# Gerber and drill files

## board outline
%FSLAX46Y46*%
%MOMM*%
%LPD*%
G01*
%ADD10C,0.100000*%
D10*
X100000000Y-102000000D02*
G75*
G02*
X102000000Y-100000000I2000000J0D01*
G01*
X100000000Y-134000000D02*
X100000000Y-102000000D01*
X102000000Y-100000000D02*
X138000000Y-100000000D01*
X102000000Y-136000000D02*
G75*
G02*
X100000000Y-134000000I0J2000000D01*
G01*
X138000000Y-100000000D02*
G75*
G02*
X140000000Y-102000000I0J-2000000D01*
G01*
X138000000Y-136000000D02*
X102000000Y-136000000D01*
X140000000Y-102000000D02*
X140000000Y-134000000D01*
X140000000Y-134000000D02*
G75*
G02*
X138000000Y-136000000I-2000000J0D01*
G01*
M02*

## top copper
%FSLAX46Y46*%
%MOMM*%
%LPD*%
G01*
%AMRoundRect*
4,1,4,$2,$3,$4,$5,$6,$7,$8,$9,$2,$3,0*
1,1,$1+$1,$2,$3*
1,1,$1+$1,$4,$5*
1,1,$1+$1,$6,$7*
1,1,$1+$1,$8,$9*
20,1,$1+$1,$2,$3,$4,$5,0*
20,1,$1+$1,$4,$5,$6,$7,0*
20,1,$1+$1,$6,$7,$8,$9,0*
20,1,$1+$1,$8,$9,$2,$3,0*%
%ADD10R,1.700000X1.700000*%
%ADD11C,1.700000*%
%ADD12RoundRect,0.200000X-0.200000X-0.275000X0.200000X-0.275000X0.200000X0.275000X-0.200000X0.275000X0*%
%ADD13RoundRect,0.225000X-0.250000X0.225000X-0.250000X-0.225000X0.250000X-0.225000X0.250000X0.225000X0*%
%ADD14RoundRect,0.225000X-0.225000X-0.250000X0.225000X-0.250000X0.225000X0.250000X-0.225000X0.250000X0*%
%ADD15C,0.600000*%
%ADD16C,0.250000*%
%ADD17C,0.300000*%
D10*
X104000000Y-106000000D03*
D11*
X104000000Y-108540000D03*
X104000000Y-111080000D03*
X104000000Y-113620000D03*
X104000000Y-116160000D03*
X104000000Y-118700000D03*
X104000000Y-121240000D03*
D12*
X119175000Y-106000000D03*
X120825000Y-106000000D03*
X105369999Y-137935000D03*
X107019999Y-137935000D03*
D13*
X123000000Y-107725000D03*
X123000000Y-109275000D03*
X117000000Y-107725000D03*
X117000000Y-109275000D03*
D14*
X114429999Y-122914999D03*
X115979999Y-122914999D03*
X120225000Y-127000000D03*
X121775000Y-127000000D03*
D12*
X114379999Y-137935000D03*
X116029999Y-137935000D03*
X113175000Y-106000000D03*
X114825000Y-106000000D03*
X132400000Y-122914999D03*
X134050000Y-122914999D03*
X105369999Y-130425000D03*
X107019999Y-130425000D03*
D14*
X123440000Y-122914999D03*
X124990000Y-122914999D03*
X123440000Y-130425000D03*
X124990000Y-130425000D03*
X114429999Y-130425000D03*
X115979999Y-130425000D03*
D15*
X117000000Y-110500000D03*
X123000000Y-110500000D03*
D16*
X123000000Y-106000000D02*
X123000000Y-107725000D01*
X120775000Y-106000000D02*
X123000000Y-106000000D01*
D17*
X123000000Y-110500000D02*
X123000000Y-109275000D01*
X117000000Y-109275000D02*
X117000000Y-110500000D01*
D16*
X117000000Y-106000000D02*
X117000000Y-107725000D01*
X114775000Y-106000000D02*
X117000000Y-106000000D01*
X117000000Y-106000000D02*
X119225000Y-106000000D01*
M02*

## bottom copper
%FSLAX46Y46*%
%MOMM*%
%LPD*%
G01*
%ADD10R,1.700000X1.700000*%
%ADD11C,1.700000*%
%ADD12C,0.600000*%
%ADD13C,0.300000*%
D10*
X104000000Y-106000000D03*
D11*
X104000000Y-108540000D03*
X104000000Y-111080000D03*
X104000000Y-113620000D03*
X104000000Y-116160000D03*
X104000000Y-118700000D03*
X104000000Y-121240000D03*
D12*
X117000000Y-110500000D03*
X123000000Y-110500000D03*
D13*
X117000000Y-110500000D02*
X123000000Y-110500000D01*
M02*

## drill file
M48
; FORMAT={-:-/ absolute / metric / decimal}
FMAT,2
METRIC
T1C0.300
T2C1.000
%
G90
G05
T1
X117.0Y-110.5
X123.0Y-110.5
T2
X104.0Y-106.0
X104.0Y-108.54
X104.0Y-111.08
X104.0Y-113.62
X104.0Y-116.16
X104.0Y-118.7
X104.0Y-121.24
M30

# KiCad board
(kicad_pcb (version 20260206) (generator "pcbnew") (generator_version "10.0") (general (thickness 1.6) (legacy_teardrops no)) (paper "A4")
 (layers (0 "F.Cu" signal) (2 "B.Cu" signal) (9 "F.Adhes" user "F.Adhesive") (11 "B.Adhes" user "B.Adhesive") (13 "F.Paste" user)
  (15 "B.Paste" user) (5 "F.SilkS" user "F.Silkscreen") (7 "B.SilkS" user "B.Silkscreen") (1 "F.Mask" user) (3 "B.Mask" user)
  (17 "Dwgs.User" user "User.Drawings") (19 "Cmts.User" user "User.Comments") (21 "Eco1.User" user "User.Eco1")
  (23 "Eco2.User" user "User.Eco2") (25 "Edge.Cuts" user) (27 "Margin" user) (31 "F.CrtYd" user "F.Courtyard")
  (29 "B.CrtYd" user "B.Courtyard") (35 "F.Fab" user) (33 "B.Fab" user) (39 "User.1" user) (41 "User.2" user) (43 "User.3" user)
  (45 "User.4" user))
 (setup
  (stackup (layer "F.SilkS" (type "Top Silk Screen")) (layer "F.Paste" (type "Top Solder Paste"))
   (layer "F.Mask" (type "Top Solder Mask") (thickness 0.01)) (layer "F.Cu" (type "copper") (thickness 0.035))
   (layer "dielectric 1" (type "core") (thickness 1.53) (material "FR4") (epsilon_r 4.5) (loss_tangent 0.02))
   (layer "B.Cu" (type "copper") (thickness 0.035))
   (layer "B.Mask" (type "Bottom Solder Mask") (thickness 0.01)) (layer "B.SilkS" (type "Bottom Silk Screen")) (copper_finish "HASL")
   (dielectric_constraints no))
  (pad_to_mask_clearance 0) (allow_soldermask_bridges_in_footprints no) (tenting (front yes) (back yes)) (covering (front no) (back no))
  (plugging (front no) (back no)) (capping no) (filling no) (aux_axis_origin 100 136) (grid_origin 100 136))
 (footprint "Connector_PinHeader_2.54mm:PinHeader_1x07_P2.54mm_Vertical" (layer "F.Cu") (at 104 106)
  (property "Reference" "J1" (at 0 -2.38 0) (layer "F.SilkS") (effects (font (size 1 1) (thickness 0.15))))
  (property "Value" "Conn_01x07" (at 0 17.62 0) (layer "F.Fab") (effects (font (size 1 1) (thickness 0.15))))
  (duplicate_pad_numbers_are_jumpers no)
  (pad "1" thru_hole rect (at 0 0) (size 1.7 1.7) (drill 1) (layers "*.Cu" "*.Mask") (remove_unused_layers no) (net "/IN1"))
  (pad "2" thru_hole circle (at 0 2.54) (size 1.7 1.7) (drill 1) (layers "*.Cu" "*.Mask") (remove_unused_layers no) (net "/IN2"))
  (pad "3" thru_hole circle (at 0 5.08) (size 1.7 1.7) (drill 1) (layers "*.Cu" "*.Mask") (remove_unused_layers no) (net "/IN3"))
  (pad "4" thru_hole circle (at 0 7.62) (size 1.7 1.7) (drill 1) (layers "*.Cu" "*.Mask") (remove_unused_layers no) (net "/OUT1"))
  (pad "5" thru_hole circle (at 0 10.16) (size 1.7 1.7) (drill 1) (layers "*.Cu" "*.Mask") (remove_unused_layers no) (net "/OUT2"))
  (pad "6" thru_hole circle (at 0 12.7) (size 1.7 1.7) (drill 1) (layers "*.Cu" "*.Mask") (remove_unused_layers no) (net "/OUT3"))
  (pad "7" thru_hole circle (at 0 15.24) (size 1.7 1.7) (drill 1) (layers "*.Cu" "*.Mask") (remove_unused_layers no) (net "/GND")))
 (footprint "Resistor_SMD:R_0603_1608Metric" (layer "F.Cu") (at 120 106)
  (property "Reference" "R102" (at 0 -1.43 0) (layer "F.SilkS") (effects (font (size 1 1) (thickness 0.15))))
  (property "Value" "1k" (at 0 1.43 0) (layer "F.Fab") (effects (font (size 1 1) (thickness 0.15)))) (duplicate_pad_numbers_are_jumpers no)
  (pad "1" smd roundrect (at -0.825 0) (size 0.8 0.95) (layers "F.Cu" "F.Mask" "F.Paste") (roundrect_rratio 0.25) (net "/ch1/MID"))
  (pad "2" smd roundrect (at 0.825 0) (size 0.8 0.95) (layers "F.Cu" "F.Mask" "F.Paste") (roundrect_rratio 0.25) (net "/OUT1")))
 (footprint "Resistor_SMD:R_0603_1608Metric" (layer "F.Cu") (at 106.194999 137.935)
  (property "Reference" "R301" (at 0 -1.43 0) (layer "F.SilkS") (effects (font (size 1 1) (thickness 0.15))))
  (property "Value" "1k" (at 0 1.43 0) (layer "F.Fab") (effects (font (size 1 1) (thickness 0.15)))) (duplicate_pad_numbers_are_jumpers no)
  (pad "1" smd roundrect (at -0.825 0) (size 0.8 0.95) (layers "F.Cu" "F.Mask" "F.Paste") (roundrect_rratio 0.25) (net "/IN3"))
  (pad "2" smd roundrect (at 0.825 0) (size 0.8 0.95) (layers "F.Cu" "F.Mask" "F.Paste") (roundrect_rratio 0.25) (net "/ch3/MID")))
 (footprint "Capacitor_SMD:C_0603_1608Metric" (layer "F.Cu") (at 123 108.5 -90)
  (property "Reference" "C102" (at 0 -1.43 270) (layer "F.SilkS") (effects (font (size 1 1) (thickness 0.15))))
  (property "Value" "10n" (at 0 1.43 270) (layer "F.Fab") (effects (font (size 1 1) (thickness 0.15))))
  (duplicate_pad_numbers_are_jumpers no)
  (pad "1" smd roundrect (at -0.775 0 270) (size 0.9 0.95) (layers "F.Cu" "F.Mask" "F.Paste") (roundrect_rratio 0.25) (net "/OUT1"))
  (pad "2" smd roundrect (at 0.775 0 270) (size 0.9 0.95) (layers "F.Cu" "F.Mask" "F.Paste") (roundrect_rratio 0.25) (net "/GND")))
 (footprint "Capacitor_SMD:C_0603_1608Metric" (layer "F.Cu") (at 117 108.5 -90)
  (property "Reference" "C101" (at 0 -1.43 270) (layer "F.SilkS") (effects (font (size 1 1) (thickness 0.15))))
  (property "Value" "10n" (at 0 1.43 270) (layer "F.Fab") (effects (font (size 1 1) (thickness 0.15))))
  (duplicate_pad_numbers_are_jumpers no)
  (pad "1" smd roundrect (at -0.775 0 270) (size 0.9 0.95) (layers "F.Cu" "F.Mask" "F.Paste") (roundrect_rratio 0.25) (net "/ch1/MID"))
  (pad "2" smd roundrect (at 0.775 0 270) (size 0.9 0.95) (layers "F.Cu" "F.Mask" "F.Paste") (roundrect_rratio 0.25) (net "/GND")))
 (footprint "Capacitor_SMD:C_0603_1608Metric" (layer "F.Cu") (at 115.204999 122.914999)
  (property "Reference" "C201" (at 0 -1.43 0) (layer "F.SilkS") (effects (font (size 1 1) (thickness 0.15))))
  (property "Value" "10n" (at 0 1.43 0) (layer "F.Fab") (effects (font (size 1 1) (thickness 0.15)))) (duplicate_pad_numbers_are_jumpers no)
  (pad "1" smd roundrect (at -0.775 0) (size 0.9 0.95) (layers "F.Cu" "F.Mask" "F.Paste") (roundrect_rratio 0.25) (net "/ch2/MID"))
  (pad "2" smd roundrect (at 0.775 0) (size 0.9 0.95) (layers "F.Cu" "F.Mask" "F.Paste") (roundrect_rratio 0.25) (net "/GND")))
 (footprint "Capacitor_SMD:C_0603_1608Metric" (layer "F.Cu") (at 121 127)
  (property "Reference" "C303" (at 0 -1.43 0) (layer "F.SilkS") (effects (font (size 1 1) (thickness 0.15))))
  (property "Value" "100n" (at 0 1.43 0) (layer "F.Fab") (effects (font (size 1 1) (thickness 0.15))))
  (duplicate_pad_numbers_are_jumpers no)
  (pad "1" smd roundrect (at -0.775 0) (size 0.9 0.95) (layers "F.Cu" "F.Mask" "F.Paste") (roundrect_rratio 0.25) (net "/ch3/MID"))
  (pad "2" smd roundrect (at 0.775 0) (size 0.9 0.95) (layers "F.Cu" "F.Mask" "F.Paste") (roundrect_rratio 0.25) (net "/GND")))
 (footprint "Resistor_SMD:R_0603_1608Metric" (layer "F.Cu") (at 115.204999 137.935)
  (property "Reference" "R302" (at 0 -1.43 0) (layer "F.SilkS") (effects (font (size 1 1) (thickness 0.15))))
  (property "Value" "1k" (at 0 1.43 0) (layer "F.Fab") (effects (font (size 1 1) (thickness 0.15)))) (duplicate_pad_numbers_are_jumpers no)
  (pad "1" smd roundrect (at -0.825 0) (size 0.8 0.95) (layers "F.Cu" "F.Mask" "F.Paste") (roundrect_rratio 0.25) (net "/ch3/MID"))
  (pad "2" smd roundrect (at 0.825 0) (size 0.8 0.95) (layers "F.Cu" "F.Mask" "F.Paste") (roundrect_rratio 0.25) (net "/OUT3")))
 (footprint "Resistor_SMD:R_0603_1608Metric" (layer "F.Cu") (at 114 106)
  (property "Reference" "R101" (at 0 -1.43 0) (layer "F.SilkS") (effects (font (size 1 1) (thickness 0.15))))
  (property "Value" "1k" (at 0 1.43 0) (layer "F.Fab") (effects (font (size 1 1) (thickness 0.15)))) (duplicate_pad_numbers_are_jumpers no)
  (pad "1" smd roundrect (at -0.825 0) (size 0.8 0.95) (layers "F.Cu" "F.Mask" "F.Paste") (roundrect_rratio 0.25) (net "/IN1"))
  (pad "2" smd roundrect (at 0.825 0) (size 0.8 0.95) (layers "F.Cu" "F.Mask" "F.Paste") (roundrect_rratio 0.25) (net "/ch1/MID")))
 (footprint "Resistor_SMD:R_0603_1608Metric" (layer "F.Cu") (at 133.225 122.914999)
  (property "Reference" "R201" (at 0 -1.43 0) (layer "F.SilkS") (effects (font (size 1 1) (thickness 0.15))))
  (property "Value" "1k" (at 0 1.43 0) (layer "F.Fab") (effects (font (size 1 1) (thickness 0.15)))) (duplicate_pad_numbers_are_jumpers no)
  (pad "1" smd roundrect (at -0.825 0) (size 0.8 0.95) (layers "F.Cu" "F.Mask" "F.Paste") (roundrect_rratio 0.25) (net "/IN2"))
  (pad "2" smd roundrect (at 0.825 0) (size 0.8 0.95) (layers "F.Cu" "F.Mask" "F.Paste") (roundrect_rratio 0.25) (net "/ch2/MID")))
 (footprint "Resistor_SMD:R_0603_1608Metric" (layer "F.Cu") (at 106.194999 130.425)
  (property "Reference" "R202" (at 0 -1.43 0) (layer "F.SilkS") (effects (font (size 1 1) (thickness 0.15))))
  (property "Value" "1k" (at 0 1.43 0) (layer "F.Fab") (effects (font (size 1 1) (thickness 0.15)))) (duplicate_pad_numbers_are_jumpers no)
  (pad "1" smd roundrect (at -0.825 0) (size 0.8 0.95) (layers "F.Cu" "F.Mask" "F.Paste") (roundrect_rratio 0.25) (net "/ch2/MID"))
  (pad "2" smd roundrect (at 0.825 0) (size 0.8 0.95) (layers "F.Cu" "F.Mask" "F.Paste") (roundrect_rratio 0.25) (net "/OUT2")))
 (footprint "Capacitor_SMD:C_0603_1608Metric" (layer "F.Cu") (at 124.215 122.914999)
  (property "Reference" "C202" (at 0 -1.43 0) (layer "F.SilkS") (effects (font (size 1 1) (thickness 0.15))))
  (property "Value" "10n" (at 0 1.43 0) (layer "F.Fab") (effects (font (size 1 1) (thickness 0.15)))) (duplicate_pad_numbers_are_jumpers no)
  (pad "1" smd roundrect (at -0.775 0) (size 0.9 0.95) (layers "F.Cu" "F.Mask" "F.Paste") (roundrect_rratio 0.25) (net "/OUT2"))
  (pad "2" smd roundrect (at 0.775 0) (size 0.9 0.95) (layers "F.Cu" "F.Mask" "F.Paste") (roundrect_rratio 0.25) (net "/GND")))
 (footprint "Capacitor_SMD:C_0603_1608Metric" (layer "F.Cu") (at 124.215 130.425)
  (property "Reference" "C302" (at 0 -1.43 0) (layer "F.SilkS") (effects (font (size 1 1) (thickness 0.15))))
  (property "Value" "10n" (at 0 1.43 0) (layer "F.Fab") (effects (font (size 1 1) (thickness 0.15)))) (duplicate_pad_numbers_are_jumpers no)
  (pad "1" smd roundrect (at -0.775 0) (size 0.9 0.95) (layers "F.Cu" "F.Mask" "F.Paste") (roundrect_rratio 0.25) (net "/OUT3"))
  (pad "2" smd roundrect (at 0.775 0) (size 0.9 0.95) (layers "F.Cu" "F.Mask" "F.Paste") (roundrect_rratio 0.25) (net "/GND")))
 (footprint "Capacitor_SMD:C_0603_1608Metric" (layer "F.Cu") (at 115.204999 130.425)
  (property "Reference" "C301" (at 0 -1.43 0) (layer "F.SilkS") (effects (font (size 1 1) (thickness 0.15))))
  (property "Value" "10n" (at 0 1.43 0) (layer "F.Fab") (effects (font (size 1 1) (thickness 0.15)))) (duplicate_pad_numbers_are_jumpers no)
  (pad "1" smd roundrect (at -0.775 0) (size 0.9 0.95) (layers "F.Cu" "F.Mask" "F.Paste") (roundrect_rratio 0.25) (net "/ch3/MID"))
  (pad "2" smd roundrect (at 0.775 0) (size 0.9 0.95) (layers "F.Cu" "F.Mask" "F.Paste") (roundrect_rratio 0.25) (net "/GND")))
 (gr_arc (start 100 102) (mid 100.585786 100.585786) (end 102 100) (stroke (width 0.1) (type default)) (layer "Edge.Cuts"))
 (gr_line (start 100 134) (end 100 102) (stroke (width 0.1) (type default)) (layer "Edge.Cuts"))
 (gr_line (start 102 100) (end 138 100) (stroke (width 0.1) (type default)) (layer "Edge.Cuts"))
 (gr_arc (start 102 136) (mid 100.585786 135.414213) (end 100 134) (stroke (width 0.1) (type default)) (layer "Edge.Cuts"))
 (gr_arc (start 138 100) (mid 139.414213 100.585786) (end 140 102) (stroke (width 0.1) (type default)) (layer "Edge.Cuts"))
 (gr_line (start 138 136) (end 102 136) (stroke (width 0.1) (type default)) (layer "Edge.Cuts"))
 (gr_line (start 140 102) (end 140 134) (stroke (width 0.1) (type default)) (layer "Edge.Cuts"))
 (gr_arc (start 140 134) (mid 139.414213 135.414213) (end 138 136) (stroke (width 0.1) (type default)) (layer "Edge.Cuts"))
 (segment (start 123 106) (end 123 107.725) (width 0.25) (layer "F.Cu") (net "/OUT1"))
 (segment (start 120.775 106) (end 123 106) (width 0.25) (layer "F.Cu") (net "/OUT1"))
 (segment (start 123 110.5) (end 123 109.275) (width 0.3) (layer "F.Cu") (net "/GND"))
 (segment (start 117 109.275) (end 117 110.5) (width 0.3) (layer "F.Cu") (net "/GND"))
 (via (at 117 110.5) (size 0.6) (drill 0.3) (layers "F.Cu" "B.Cu") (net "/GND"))
 (via (at 123 110.5) (size 0.6) (drill 0.3) (layers "F.Cu" "B.Cu") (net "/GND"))
 (segment (start 117 110.5) (end 123 110.5) (width 0.3) (layer "B.Cu") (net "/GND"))
 (segment (start 117 106) (end 117 107.725) (width 0.25) (layer "F.Cu") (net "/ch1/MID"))
 (segment (start 114.775 106) (end 117 106) (width 0.25) (layer "F.Cu") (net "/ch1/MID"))
 (segment (start 117 106) (end 119.225 106) (width 0.25) (layer "F.Cu") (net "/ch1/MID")))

